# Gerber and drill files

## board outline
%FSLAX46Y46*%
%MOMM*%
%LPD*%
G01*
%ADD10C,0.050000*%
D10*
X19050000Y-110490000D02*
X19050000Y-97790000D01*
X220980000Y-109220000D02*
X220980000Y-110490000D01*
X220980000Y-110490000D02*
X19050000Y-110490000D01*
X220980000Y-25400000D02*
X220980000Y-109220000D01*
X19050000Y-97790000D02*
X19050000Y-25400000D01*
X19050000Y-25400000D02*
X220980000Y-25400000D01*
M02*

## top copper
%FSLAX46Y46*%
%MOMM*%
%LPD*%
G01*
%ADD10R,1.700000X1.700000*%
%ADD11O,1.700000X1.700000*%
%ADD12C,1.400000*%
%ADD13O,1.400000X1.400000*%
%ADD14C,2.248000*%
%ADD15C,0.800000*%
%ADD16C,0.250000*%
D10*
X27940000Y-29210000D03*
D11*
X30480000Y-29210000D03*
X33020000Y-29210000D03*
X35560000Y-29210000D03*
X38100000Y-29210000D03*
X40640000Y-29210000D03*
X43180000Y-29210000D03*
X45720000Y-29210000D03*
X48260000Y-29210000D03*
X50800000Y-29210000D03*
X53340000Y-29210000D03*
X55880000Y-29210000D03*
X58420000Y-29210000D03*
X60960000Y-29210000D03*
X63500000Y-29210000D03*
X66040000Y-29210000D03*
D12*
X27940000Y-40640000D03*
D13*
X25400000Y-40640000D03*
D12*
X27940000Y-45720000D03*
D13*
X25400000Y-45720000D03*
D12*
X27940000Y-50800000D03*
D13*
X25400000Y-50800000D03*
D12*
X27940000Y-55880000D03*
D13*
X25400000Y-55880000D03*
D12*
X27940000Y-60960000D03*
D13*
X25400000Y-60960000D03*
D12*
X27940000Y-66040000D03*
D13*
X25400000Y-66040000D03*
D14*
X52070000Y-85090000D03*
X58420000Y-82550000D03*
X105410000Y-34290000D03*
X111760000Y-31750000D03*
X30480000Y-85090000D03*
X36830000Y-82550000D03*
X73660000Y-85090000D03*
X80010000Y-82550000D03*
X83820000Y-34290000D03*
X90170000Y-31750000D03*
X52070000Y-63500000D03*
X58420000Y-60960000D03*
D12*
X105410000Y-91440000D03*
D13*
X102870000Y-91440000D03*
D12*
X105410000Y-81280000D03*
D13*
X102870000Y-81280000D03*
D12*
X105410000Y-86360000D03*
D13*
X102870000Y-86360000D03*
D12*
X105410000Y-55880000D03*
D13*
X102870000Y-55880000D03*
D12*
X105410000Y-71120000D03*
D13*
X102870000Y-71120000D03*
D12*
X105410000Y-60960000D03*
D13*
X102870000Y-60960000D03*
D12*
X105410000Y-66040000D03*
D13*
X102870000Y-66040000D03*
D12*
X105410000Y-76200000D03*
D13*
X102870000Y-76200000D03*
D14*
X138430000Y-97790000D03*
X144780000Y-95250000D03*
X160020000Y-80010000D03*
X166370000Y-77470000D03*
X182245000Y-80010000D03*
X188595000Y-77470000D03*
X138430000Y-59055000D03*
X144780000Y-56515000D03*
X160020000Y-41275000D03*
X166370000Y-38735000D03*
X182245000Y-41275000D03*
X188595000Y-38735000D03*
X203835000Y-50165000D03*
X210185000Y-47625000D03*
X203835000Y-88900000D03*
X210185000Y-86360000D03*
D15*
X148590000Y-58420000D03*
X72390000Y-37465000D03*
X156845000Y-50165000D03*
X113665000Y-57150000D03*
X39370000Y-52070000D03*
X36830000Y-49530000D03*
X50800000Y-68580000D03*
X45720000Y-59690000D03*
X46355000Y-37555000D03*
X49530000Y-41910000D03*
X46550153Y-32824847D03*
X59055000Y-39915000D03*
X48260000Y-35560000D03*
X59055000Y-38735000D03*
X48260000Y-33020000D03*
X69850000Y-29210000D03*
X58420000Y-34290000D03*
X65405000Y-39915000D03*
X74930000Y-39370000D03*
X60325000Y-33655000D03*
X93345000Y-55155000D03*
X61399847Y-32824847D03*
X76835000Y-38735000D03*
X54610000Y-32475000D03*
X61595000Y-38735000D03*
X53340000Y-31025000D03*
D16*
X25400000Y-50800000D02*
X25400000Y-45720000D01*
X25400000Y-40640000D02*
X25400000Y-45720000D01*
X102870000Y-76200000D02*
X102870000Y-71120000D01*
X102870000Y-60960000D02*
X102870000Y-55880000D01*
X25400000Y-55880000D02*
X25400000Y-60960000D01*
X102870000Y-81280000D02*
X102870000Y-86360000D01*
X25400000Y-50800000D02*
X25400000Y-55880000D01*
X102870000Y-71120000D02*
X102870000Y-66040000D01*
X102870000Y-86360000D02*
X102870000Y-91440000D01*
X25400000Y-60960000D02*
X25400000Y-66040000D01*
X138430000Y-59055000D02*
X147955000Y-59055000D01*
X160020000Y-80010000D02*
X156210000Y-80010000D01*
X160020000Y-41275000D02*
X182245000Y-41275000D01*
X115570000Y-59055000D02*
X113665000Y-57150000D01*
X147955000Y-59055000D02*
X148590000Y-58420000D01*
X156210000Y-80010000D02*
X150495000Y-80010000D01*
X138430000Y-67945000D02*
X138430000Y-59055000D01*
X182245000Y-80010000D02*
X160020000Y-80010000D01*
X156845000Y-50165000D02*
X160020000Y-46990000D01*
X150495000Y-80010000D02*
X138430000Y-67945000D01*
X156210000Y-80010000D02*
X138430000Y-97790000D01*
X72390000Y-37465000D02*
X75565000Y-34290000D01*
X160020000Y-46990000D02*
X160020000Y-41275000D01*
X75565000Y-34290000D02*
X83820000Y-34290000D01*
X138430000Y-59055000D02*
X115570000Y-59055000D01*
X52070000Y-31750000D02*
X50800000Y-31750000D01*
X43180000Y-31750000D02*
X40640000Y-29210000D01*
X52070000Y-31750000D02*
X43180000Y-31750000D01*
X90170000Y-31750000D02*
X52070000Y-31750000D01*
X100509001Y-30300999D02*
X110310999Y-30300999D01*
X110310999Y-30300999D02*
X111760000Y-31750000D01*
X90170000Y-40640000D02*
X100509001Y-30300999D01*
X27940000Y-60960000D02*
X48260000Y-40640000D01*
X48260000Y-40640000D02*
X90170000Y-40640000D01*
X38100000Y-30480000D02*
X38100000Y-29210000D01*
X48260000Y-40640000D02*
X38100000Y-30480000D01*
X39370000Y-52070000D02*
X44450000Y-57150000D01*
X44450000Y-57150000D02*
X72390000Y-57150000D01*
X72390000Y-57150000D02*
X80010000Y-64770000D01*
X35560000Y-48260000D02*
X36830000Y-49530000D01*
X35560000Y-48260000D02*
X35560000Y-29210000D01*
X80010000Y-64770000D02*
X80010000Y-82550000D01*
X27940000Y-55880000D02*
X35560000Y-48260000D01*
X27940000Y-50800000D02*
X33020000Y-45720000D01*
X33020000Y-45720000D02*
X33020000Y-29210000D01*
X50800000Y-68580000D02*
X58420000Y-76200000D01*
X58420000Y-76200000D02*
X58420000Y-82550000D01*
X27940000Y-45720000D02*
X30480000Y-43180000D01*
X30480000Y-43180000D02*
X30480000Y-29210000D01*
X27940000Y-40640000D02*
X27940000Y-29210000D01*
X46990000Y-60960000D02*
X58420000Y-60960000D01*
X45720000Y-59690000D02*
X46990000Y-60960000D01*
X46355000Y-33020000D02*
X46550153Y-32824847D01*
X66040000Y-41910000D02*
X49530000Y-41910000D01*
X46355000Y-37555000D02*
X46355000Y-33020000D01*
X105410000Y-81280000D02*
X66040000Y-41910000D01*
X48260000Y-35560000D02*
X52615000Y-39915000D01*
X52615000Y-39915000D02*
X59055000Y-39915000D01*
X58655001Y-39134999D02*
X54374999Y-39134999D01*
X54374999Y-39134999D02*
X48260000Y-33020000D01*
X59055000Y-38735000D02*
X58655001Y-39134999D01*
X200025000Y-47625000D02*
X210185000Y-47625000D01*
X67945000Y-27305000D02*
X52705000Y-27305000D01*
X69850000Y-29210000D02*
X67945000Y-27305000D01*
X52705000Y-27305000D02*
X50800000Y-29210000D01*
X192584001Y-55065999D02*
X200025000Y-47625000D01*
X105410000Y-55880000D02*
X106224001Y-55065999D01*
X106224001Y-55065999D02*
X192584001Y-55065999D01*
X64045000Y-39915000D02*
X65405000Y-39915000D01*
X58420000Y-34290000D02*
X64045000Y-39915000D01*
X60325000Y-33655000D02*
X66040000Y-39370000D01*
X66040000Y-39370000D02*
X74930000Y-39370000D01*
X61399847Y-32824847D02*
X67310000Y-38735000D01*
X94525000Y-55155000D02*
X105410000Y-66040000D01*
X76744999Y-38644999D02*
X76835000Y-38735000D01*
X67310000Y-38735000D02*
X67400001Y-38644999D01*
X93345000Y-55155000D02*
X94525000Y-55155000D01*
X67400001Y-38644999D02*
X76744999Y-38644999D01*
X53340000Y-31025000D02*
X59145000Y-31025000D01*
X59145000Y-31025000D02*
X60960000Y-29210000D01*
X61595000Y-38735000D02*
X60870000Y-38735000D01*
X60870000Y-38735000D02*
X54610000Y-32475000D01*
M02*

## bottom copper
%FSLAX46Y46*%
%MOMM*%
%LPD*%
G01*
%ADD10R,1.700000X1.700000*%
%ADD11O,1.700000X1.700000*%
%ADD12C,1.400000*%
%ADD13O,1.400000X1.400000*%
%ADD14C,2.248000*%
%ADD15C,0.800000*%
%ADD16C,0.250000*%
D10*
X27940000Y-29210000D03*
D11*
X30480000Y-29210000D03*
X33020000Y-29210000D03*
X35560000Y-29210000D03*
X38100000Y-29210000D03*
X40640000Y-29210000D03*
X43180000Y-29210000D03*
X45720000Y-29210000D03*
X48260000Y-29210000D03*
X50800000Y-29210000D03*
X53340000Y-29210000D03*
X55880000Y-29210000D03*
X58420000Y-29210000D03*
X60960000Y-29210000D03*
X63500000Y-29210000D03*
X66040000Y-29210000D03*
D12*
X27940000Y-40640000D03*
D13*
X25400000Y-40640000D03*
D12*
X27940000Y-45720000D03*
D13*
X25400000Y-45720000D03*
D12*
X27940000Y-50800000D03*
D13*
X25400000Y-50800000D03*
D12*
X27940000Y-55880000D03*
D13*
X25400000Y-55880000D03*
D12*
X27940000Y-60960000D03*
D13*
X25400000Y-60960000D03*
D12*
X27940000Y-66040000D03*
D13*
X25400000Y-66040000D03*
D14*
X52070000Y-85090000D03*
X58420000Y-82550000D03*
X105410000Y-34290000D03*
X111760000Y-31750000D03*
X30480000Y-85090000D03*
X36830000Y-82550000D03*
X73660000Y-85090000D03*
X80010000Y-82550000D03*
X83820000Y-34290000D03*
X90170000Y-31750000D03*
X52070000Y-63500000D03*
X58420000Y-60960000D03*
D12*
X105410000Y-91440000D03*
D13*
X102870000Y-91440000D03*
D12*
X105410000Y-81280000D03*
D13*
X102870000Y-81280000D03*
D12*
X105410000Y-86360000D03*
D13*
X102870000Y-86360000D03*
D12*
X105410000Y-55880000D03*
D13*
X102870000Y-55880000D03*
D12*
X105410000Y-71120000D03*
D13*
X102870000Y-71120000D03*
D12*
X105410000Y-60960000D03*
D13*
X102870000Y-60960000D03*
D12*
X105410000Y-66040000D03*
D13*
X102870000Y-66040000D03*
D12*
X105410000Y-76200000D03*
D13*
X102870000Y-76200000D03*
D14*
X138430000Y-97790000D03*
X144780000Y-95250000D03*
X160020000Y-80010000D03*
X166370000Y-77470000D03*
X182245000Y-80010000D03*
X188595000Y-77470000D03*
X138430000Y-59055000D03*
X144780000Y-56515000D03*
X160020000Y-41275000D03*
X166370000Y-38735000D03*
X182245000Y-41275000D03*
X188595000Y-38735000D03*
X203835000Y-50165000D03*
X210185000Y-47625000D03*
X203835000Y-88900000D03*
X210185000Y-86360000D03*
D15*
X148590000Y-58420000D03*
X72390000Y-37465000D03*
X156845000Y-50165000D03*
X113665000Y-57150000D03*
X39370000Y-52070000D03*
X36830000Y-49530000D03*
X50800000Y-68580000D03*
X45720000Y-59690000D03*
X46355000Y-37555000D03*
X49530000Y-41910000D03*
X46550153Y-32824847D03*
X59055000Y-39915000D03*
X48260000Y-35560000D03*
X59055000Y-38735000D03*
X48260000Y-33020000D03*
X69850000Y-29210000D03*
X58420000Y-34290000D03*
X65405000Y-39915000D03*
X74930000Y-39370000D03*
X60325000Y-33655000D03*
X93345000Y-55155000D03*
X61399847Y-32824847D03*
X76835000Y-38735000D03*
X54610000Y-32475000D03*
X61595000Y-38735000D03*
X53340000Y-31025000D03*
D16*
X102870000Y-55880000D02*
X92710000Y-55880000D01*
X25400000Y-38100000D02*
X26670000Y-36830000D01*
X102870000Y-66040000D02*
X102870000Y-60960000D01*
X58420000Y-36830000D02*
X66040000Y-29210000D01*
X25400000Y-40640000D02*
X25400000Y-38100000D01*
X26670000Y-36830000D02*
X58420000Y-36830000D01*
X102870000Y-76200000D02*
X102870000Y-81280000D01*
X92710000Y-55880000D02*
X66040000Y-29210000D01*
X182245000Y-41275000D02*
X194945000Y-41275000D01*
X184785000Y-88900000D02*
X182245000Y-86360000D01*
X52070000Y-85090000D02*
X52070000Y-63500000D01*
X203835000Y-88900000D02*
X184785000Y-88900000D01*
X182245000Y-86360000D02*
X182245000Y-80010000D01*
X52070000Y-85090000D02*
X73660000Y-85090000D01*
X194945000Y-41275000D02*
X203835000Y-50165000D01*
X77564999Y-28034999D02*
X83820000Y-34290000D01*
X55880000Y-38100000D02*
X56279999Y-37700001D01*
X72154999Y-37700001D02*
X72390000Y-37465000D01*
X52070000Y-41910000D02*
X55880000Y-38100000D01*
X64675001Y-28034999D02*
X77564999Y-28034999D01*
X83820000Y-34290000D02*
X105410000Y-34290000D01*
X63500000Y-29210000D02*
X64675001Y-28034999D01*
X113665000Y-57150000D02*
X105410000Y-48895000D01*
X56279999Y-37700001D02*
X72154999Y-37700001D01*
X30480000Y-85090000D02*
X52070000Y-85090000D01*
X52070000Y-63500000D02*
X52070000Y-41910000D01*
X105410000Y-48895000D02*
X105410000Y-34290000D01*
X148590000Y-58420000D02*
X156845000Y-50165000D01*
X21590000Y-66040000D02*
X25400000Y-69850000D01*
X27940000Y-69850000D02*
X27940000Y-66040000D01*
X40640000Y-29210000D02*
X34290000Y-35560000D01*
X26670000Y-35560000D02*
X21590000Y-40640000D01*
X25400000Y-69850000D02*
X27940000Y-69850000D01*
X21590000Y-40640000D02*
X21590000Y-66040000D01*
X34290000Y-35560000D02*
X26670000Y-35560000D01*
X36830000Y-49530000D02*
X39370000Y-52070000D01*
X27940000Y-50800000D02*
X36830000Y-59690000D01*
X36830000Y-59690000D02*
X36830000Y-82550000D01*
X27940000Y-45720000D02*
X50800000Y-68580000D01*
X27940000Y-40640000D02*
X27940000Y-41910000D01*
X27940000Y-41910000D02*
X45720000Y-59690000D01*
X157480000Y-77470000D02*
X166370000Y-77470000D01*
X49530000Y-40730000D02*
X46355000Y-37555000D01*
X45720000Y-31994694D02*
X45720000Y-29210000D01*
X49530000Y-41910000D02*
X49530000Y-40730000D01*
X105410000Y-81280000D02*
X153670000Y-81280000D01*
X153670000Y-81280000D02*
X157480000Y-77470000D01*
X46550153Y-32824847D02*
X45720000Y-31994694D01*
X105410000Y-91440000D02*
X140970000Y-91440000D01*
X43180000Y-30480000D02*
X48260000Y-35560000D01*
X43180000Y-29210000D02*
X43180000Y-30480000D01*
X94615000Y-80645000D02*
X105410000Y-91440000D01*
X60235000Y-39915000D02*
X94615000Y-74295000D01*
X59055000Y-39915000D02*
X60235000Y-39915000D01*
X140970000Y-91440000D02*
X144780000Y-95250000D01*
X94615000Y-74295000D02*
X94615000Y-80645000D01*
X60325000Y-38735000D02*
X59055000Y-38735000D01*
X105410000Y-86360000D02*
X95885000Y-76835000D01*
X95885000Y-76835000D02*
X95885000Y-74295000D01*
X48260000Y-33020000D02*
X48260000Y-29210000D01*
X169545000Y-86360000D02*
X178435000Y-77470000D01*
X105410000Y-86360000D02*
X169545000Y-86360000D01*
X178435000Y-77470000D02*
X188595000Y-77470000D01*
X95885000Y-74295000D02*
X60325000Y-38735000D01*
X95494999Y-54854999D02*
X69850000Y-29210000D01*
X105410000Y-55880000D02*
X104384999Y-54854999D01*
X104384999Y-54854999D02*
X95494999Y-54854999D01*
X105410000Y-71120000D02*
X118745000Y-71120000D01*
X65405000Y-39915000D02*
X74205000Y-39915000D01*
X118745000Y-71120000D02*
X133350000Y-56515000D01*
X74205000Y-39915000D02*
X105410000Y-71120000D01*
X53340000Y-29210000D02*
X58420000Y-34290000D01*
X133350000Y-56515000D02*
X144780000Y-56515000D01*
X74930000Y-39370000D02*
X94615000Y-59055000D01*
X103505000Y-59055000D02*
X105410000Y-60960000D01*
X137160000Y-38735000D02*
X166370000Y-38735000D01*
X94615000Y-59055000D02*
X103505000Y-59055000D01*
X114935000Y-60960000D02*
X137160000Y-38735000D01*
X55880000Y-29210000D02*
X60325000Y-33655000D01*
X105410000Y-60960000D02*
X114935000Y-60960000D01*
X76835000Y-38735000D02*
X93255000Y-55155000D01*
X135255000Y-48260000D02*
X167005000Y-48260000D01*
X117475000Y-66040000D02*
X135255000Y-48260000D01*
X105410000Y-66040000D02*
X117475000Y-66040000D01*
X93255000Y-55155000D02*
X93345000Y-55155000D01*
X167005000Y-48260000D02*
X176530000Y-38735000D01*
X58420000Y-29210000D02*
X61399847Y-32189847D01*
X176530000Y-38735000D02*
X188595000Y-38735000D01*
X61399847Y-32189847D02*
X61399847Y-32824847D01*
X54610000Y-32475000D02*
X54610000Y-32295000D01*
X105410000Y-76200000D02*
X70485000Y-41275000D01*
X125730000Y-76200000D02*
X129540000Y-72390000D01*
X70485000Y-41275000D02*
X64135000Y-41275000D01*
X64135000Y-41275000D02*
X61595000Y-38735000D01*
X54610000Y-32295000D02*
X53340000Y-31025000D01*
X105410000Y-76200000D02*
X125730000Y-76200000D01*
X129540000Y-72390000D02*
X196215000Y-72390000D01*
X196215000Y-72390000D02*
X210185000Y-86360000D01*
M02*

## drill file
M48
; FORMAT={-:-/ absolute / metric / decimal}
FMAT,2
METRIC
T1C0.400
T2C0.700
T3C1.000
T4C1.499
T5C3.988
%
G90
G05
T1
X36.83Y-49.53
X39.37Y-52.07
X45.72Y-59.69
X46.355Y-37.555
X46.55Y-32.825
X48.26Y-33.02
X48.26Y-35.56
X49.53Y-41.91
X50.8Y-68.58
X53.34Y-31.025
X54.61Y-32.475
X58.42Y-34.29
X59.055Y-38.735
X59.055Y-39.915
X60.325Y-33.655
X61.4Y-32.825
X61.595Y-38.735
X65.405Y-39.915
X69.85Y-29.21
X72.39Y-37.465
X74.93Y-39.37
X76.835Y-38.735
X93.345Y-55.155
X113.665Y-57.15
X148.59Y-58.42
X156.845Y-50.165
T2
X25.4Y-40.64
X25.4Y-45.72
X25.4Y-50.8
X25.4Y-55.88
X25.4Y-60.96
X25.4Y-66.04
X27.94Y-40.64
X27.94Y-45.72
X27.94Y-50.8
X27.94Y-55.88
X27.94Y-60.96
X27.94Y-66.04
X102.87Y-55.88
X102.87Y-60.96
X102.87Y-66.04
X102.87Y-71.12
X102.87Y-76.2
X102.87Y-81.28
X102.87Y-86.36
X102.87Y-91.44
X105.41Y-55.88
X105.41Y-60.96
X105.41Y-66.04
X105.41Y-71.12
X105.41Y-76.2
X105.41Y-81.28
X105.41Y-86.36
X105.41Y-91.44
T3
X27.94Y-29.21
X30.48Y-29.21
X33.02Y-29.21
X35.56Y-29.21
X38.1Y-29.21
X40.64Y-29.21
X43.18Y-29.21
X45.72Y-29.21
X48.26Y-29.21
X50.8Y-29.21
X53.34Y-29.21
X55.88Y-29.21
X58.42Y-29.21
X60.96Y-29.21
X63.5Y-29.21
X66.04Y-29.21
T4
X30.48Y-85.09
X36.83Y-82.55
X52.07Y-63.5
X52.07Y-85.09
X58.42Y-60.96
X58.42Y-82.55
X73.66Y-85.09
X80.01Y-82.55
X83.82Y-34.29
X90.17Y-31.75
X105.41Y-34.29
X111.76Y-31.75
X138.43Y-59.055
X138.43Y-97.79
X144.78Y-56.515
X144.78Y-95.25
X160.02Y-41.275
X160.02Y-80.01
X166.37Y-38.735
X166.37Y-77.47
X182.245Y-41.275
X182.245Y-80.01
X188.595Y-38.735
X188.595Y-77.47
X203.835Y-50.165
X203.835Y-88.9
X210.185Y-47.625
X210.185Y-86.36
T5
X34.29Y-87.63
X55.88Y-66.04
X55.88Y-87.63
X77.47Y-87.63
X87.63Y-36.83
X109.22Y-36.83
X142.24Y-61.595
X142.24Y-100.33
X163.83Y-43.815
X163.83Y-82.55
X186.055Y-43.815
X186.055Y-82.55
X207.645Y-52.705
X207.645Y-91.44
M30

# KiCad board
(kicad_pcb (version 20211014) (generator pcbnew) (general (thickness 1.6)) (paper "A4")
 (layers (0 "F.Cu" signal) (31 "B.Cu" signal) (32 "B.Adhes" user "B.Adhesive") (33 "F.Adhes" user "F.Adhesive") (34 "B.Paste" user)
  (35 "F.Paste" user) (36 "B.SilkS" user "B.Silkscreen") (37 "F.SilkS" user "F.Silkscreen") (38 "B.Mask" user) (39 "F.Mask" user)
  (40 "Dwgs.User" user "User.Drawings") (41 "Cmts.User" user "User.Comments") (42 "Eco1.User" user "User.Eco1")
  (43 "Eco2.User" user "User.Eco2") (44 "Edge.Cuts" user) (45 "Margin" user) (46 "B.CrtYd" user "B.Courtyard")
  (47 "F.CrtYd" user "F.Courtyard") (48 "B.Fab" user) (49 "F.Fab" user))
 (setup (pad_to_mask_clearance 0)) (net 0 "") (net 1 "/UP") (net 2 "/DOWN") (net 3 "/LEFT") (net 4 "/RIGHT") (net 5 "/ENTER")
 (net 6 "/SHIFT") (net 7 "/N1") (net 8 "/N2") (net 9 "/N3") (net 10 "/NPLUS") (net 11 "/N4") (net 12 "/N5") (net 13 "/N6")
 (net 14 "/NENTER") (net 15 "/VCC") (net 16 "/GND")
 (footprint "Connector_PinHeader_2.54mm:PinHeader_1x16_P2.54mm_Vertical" (layer "F.Cu") (at 27.94 29.21 90)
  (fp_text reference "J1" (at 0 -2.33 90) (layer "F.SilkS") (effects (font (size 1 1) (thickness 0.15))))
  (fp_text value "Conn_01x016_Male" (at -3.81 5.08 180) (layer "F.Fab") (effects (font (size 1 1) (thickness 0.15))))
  (pad "1" thru_hole rect locked (at 0 0 90) (size 1.7 1.7) (drill 1) (layers *.Cu *.Mask) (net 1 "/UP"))
  (pad "2" thru_hole oval locked (at 0 2.54 90) (size 1.7 1.7) (drill 1) (layers *.Cu *.Mask) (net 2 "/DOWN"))
  (pad "3" thru_hole oval locked (at 0 5.08 90) (size 1.7 1.7) (drill 1) (layers *.Cu *.Mask) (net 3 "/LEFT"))
  (pad "4" thru_hole oval locked (at 0 7.62 90) (size 1.7 1.7) (drill 1) (layers *.Cu *.Mask) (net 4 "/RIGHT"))
  (pad "5" thru_hole oval locked (at 0 10.16 90) (size 1.7 1.7) (drill 1) (layers *.Cu *.Mask) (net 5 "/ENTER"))
  (pad "6" thru_hole oval locked (at 0 12.7 90) (size 1.7 1.7) (drill 1) (layers *.Cu *.Mask) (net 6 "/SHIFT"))
  (pad "7" thru_hole oval locked (at 0 15.24 90) (size 1.7 1.7) (drill 1) (layers *.Cu *.Mask) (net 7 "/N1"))
  (pad "8" thru_hole oval locked (at 0 17.78 90) (size 1.7 1.7) (drill 1) (layers *.Cu *.Mask) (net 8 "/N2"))
  (pad "9" thru_hole oval locked (at 0 20.32 90) (size 1.7 1.7) (drill 1) (layers *.Cu *.Mask) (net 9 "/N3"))
  (pad "10" thru_hole oval locked (at 0 22.86 90) (size 1.7 1.7) (drill 1) (layers *.Cu *.Mask) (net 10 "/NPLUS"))
  (pad "11" thru_hole oval locked (at 0 25.4 90) (size 1.7 1.7) (drill 1) (layers *.Cu *.Mask) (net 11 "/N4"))
  (pad "12" thru_hole oval locked (at 0 27.94 90) (size 1.7 1.7) (drill 1) (layers *.Cu *.Mask) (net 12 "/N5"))
  (pad "13" thru_hole oval locked (at 0 30.48 90) (size 1.7 1.7) (drill 1) (layers *.Cu *.Mask) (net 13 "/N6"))
  (pad "14" thru_hole oval locked (at 0 33.02 90) (size 1.7 1.7) (drill 1) (layers *.Cu *.Mask) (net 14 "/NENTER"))
  (pad "15" thru_hole oval locked (at 0 35.56 90) (size 1.7 1.7) (drill 1) (layers *.Cu *.Mask) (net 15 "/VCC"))
  (pad "16" thru_hole oval locked (at 0 38.1 90) (size 1.7 1.7) (drill 1) (layers *.Cu *.Mask) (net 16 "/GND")))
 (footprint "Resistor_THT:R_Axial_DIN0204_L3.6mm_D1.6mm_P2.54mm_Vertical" (layer "F.Cu") (at 27.94 40.64 180)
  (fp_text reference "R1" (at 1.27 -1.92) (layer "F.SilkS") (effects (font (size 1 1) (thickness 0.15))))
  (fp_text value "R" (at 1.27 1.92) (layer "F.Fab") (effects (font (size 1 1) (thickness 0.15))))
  (pad "1" thru_hole circle locked (at 0 0 180) (size 1.4 1.4) (drill 0.7) (layers *.Cu *.Mask) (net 1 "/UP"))
  (pad "2" thru_hole oval locked (at 2.54 0 180) (size 1.4 1.4) (drill 0.7) (layers *.Cu *.Mask) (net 16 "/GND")))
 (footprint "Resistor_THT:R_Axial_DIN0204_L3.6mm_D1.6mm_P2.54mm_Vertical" (layer "F.Cu") (at 27.94 45.72 180)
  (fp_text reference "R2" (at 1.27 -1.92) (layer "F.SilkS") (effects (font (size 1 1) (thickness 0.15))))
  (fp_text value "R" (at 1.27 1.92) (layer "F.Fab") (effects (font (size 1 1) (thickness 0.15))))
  (pad "1" thru_hole circle locked (at 0 0 180) (size 1.4 1.4) (drill 0.7) (layers *.Cu *.Mask) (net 2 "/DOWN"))
  (pad "2" thru_hole oval locked (at 2.54 0 180) (size 1.4 1.4) (drill 0.7) (layers *.Cu *.Mask) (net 16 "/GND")))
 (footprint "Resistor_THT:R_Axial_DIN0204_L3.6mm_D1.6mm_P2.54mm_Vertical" (layer "F.Cu") (at 27.94 50.8 180)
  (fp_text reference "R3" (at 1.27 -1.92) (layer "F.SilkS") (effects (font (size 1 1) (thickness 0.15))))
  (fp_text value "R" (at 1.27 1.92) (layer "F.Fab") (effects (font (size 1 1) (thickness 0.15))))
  (pad "1" thru_hole circle locked (at 0 0 180) (size 1.4 1.4) (drill 0.7) (layers *.Cu *.Mask) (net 3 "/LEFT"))
  (pad "2" thru_hole oval locked (at 2.54 0 180) (size 1.4 1.4) (drill 0.7) (layers *.Cu *.Mask) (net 16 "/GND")))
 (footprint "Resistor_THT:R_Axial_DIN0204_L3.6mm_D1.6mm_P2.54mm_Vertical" (layer "F.Cu") (at 27.94 55.88 180)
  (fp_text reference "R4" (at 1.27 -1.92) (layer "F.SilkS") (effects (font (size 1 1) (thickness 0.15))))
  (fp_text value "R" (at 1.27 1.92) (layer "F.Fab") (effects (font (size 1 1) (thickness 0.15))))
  (pad "1" thru_hole circle locked (at 0 0 180) (size 1.4 1.4) (drill 0.7) (layers *.Cu *.Mask) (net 4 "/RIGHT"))
  (pad "2" thru_hole oval locked (at 2.54 0 180) (size 1.4 1.4) (drill 0.7) (layers *.Cu *.Mask) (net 16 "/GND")))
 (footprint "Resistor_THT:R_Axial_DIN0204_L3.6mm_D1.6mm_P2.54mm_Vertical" (layer "F.Cu") (at 27.94 60.96 180)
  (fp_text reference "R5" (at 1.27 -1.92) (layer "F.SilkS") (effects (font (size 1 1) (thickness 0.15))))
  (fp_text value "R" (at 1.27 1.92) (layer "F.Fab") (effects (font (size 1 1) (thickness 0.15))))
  (pad "1" thru_hole circle locked (at 0 0 180) (size 1.4 1.4) (drill 0.7) (layers *.Cu *.Mask) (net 5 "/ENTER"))
  (pad "2" thru_hole oval locked (at 2.54 0 180) (size 1.4 1.4) (drill 0.7) (layers *.Cu *.Mask) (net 16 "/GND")))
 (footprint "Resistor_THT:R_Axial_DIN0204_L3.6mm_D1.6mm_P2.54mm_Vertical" (layer "F.Cu") (at 27.94 66.04 180)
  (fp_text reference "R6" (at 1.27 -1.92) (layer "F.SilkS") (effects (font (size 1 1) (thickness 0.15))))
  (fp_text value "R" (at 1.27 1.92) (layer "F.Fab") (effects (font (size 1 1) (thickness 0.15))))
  (pad "1" thru_hole circle locked (at 0 0 180) (size 1.4 1.4) (drill 0.7) (layers *.Cu *.Mask) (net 6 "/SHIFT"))
  (pad "2" thru_hole oval locked (at 2.54 0 180) (size 1.4 1.4) (drill 0.7) (layers *.Cu *.Mask) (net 16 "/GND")))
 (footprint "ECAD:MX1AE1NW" (layer "F.Cu") (at 52.07 85.09)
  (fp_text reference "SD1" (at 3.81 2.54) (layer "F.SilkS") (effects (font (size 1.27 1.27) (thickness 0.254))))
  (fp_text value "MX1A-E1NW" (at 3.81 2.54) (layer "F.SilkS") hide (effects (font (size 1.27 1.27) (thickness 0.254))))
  (pad "" np_thru_hole circle locked (at 3.81 2.54) (size 3.9878 0) (drill 3.9878) (layers *.Cu *.Mask))
  (pad "1" thru_hole circle locked (at 0 0) (size 2.248 2.248) (drill 1.4986) (layers *.Cu *.Mask) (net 15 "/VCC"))
  (pad "2" thru_hole circle locked (at 6.35 -2.54) (size 2.248 2.248) (drill 1.4986) (layers *.Cu *.Mask) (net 2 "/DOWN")))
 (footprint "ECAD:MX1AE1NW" (layer "F.Cu") (at 105.41 34.29)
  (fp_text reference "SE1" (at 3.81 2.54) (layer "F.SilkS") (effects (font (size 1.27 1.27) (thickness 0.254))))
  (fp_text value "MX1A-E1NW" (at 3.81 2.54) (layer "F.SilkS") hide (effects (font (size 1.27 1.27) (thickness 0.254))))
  (pad "" np_thru_hole circle locked (at 3.81 2.54) (size 3.9878 0) (drill 3.9878) (layers *.Cu *.Mask))
  (pad "1" thru_hole circle locked (at 0 0) (size 2.248 2.248) (drill 1.4986) (layers *.Cu *.Mask) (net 15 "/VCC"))
  (pad "2" thru_hole circle locked (at 6.35 -2.54) (size 2.248 2.248) (drill 1.4986) (layers *.Cu *.Mask) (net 5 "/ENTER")))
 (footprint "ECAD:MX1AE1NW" (layer "F.Cu") (at 30.48 85.09)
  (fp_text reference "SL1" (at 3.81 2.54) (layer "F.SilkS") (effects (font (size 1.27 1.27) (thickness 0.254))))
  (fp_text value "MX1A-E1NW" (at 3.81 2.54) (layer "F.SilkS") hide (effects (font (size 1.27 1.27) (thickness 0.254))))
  (pad "" np_thru_hole circle locked (at 3.81 2.54) (size 3.9878 0) (drill 3.9878) (layers *.Cu *.Mask))
  (pad "1" thru_hole circle locked (at 0 0) (size 2.248 2.248) (drill 1.4986) (layers *.Cu *.Mask) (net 15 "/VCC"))
  (pad "2" thru_hole circle locked (at 6.35 -2.54) (size 2.248 2.248) (drill 1.4986) (layers *.Cu *.Mask) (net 3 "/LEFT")))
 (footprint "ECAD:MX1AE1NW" (layer "F.Cu") (at 73.66 85.09)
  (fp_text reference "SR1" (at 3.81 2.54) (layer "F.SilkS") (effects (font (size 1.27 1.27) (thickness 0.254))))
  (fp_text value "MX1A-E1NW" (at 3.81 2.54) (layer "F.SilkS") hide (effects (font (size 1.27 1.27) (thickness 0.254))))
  (pad "" np_thru_hole circle locked (at 3.81 2.54) (size 3.9878 0) (drill 3.9878) (layers *.Cu *.Mask))
  (pad "1" thru_hole circle locked (at 0 0) (size 2.248 2.248) (drill 1.4986) (layers *.Cu *.Mask) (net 15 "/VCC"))
  (pad "2" thru_hole circle locked (at 6.35 -2.54) (size 2.248 2.248) (drill 1.4986) (layers *.Cu *.Mask) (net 4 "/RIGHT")))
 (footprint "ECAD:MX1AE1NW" (layer "F.Cu") (at 83.82 34.29)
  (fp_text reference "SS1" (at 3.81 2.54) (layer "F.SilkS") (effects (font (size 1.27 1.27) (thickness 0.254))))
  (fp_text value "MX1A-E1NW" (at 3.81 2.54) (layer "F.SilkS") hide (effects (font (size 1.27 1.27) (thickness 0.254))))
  (pad "" np_thru_hole circle locked (at 3.81 2.54) (size 3.9878 0) (drill 3.9878) (layers *.Cu *.Mask))
  (pad "1" thru_hole circle locked (at 0 0) (size 2.248 2.248) (drill 1.4986) (layers *.Cu *.Mask) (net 15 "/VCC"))
  (pad "2" thru_hole circle locked (at 6.35 -2.54) (size 2.248 2.248) (drill 1.4986) (layers *.Cu *.Mask) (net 6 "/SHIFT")))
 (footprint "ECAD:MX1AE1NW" (layer "F.Cu") (at 52.07 63.5)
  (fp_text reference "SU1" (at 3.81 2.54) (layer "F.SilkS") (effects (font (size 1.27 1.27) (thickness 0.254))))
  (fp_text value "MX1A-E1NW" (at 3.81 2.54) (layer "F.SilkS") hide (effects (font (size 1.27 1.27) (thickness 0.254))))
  (pad "" np_thru_hole circle locked (at 3.81 2.54) (size 3.9878 0) (drill 3.9878) (layers *.Cu *.Mask))
  (pad "1" thru_hole circle locked (at 0 0) (size 2.248 2.248) (drill 1.4986) (layers *.Cu *.Mask) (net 15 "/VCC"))
  (pad "2" thru_hole circle locked (at 6.35 -2.54) (size 2.248 2.248) (drill 1.4986) (layers *.Cu *.Mask) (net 1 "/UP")))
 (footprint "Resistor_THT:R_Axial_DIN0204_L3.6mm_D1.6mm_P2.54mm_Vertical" (layer "F.Cu") (at 105.41 91.44 180)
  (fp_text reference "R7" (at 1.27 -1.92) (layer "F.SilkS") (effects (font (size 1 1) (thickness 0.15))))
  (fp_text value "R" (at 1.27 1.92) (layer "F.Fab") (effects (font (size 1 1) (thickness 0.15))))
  (pad "1" thru_hole circle locked (at 0 0 180) (size 1.4 1.4) (drill 0.7) (layers *.Cu *.Mask) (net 7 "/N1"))
  (pad "2" thru_hole oval locked (at 2.54 0 180) (size 1.4 1.4) (drill 0.7) (layers *.Cu *.Mask) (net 16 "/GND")))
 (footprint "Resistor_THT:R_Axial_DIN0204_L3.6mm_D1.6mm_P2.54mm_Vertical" (layer "F.Cu") (at 105.41 81.28 180)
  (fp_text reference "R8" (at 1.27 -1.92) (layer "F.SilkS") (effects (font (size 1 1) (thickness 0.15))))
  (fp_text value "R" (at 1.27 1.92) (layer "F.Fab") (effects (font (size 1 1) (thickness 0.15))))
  (pad "1" thru_hole circle locked (at 0 0 180) (size 1.4 1.4) (drill 0.7) (layers *.Cu *.Mask) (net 8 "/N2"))
  (pad "2" thru_hole oval locked (at 2.54 0 180) (size 1.4 1.4) (drill 0.7) (layers *.Cu *.Mask) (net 16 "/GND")))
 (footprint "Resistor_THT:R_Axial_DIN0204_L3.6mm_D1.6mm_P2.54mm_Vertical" (layer "F.Cu") (at 105.41 86.36 180)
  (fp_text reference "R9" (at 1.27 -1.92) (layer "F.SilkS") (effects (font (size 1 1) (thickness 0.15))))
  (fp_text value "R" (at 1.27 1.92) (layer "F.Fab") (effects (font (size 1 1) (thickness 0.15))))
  (pad "1" thru_hole circle locked (at 0 0 180) (size 1.4 1.4) (drill 0.7) (layers *.Cu *.Mask) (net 9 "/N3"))
  (pad "2" thru_hole oval locked (at 2.54 0 180) (size 1.4 1.4) (drill 0.7) (layers *.Cu *.Mask) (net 16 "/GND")))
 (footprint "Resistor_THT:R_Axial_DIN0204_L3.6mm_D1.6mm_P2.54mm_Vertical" (layer "F.Cu") (at 105.41 55.88 180)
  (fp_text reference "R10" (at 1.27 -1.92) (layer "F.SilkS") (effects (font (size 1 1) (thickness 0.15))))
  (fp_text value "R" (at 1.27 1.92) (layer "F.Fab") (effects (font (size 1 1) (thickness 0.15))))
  (pad "1" thru_hole circle locked (at 0 0 180) (size 1.4 1.4) (drill 0.7) (layers *.Cu *.Mask) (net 10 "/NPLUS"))
  (pad "2" thru_hole oval locked (at 2.54 0 180) (size 1.4 1.4) (drill 0.7) (layers *.Cu *.Mask) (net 16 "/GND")))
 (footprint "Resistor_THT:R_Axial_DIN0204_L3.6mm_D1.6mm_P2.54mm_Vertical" (layer "F.Cu") (at 105.41 71.12 180)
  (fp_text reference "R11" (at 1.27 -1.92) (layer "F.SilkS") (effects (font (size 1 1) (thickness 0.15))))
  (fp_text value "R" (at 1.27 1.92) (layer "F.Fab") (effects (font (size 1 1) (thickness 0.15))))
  (pad "1" thru_hole circle locked (at 0 0 180) (size 1.4 1.4) (drill 0.7) (layers *.Cu *.Mask) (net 11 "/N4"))
  (pad "2" thru_hole oval locked (at 2.54 0 180) (size 1.4 1.4) (drill 0.7) (layers *.Cu *.Mask) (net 16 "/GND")))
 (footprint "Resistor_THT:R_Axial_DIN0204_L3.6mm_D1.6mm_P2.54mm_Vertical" (layer "F.Cu") (at 105.41 60.96 180)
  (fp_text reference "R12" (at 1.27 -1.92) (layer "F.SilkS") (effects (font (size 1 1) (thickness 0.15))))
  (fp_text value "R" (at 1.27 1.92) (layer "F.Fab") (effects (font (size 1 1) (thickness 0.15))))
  (pad "1" thru_hole circle locked (at 0 0 180) (size 1.4 1.4) (drill 0.7) (layers *.Cu *.Mask) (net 12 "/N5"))
  (pad "2" thru_hole oval locked (at 2.54 0 180) (size 1.4 1.4) (drill 0.7) (layers *.Cu *.Mask) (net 16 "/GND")))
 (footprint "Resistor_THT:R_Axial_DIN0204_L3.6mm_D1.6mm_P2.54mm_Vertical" (layer "F.Cu") (at 105.41 66.04 180)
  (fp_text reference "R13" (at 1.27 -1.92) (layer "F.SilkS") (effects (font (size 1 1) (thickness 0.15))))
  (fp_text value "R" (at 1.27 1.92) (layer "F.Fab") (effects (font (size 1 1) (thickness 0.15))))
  (pad "1" thru_hole circle locked (at 0 0 180) (size 1.4 1.4) (drill 0.7) (layers *.Cu *.Mask) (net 13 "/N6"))
  (pad "2" thru_hole oval locked (at 2.54 0 180) (size 1.4 1.4) (drill 0.7) (layers *.Cu *.Mask) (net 16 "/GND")))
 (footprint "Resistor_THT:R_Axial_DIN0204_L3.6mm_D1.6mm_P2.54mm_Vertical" (layer "F.Cu") (at 105.41 76.2 180)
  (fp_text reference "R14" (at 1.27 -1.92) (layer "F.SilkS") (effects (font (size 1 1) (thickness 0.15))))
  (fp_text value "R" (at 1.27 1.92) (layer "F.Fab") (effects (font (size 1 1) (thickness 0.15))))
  (pad "1" thru_hole circle locked (at 0 0 180) (size 1.4 1.4) (drill 0.7) (layers *.Cu *.Mask) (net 14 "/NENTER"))
  (pad "2" thru_hole oval locked (at 2.54 0 180) (size 1.4 1.4) (drill 0.7) (layers *.Cu *.Mask) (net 16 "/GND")))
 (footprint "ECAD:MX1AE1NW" (layer "F.Cu") (at 138.43 97.79)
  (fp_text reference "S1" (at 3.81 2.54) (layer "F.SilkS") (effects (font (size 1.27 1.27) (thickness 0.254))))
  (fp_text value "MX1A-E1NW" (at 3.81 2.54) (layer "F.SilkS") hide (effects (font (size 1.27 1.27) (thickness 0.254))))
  (pad "" np_thru_hole circle locked (at 3.81 2.54) (size 3.9878 0) (drill 3.9878) (layers *.Cu *.Mask))
  (pad "1" thru_hole circle locked (at 0 0) (size 2.248 2.248) (drill 1.4986) (layers *.Cu *.Mask) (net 15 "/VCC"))
  (pad "2" thru_hole circle locked (at 6.35 -2.54) (size 2.248 2.248) (drill 1.4986) (layers *.Cu *.Mask) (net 7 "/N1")))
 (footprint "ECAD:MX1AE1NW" (layer "F.Cu") (at 160.02 80.01)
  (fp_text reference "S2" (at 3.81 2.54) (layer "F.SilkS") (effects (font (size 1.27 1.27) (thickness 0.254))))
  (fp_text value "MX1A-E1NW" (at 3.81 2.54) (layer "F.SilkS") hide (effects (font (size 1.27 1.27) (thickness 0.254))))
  (pad "" np_thru_hole circle locked (at 3.81 2.54) (size 3.9878 0) (drill 3.9878) (layers *.Cu *.Mask))
  (pad "1" thru_hole circle locked (at 0 0) (size 2.248 2.248) (drill 1.4986) (layers *.Cu *.Mask) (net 15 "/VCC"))
  (pad "2" thru_hole circle locked (at 6.35 -2.54) (size 2.248 2.248) (drill 1.4986) (layers *.Cu *.Mask) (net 8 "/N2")))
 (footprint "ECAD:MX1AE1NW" (layer "F.Cu") (at 182.245 80.01)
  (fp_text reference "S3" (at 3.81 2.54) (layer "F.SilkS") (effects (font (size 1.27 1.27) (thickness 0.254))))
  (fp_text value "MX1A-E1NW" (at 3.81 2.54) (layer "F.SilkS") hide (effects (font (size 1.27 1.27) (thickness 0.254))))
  (pad "" np_thru_hole circle locked (at 3.81 2.54) (size 3.9878 0) (drill 3.9878) (layers *.Cu *.Mask))
  (pad "1" thru_hole circle locked (at 0 0) (size 2.248 2.248) (drill 1.4986) (layers *.Cu *.Mask) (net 15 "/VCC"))
  (pad "2" thru_hole circle locked (at 6.35 -2.54) (size 2.248 2.248) (drill 1.4986) (layers *.Cu *.Mask) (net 9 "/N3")))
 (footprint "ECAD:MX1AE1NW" (layer "F.Cu") (at 138.43 59.055)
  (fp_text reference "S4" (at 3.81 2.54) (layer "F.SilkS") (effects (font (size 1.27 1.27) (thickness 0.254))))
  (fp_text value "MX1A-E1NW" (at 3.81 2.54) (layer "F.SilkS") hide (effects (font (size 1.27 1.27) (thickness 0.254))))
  (pad "" np_thru_hole circle locked (at 3.81 2.54) (size 3.9878 0) (drill 3.9878) (layers *.Cu *.Mask))
  (pad "1" thru_hole circle locked (at 0 0) (size 2.248 2.248) (drill 1.4986) (layers *.Cu *.Mask) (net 15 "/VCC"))
  (pad "2" thru_hole circle locked (at 6.35 -2.54) (size 2.248 2.248) (drill 1.4986) (layers *.Cu *.Mask) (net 11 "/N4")))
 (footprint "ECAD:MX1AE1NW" (layer "F.Cu") (at 160.02 41.275)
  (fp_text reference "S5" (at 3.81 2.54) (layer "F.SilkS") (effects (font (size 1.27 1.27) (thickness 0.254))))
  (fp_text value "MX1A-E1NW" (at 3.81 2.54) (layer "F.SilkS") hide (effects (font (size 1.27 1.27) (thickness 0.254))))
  (pad "" np_thru_hole circle locked (at 3.81 2.54) (size 3.9878 0) (drill 3.9878) (layers *.Cu *.Mask))
  (pad "1" thru_hole circle locked (at 0 0) (size 2.248 2.248) (drill 1.4986) (layers *.Cu *.Mask) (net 15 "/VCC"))
  (pad "2" thru_hole circle locked (at 6.35 -2.54) (size 2.248 2.248) (drill 1.4986) (layers *.Cu *.Mask) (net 12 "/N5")))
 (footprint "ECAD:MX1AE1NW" (layer "F.Cu") (at 182.245 41.275)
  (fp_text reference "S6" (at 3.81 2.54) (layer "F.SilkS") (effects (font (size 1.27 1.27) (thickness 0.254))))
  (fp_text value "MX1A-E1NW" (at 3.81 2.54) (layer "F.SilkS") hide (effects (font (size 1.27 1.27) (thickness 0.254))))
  (pad "" np_thru_hole circle locked (at 3.81 2.54) (size 3.9878 0) (drill 3.9878) (layers *.Cu *.Mask))
  (pad "1" thru_hole circle locked (at 0 0) (size 2.248 2.248) (drill 1.4986) (layers *.Cu *.Mask) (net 15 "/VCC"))
  (pad "2" thru_hole circle locked (at 6.35 -2.54) (size 2.248 2.248) (drill 1.4986) (layers *.Cu *.Mask) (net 13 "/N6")))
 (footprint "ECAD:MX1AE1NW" (layer "F.Cu") (at 203.835 50.165)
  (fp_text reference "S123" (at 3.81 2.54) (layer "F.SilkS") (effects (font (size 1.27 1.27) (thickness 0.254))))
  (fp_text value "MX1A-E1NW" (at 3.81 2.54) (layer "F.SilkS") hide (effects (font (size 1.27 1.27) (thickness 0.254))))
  (pad "" np_thru_hole circle locked (at 3.81 2.54) (size 3.9878 0) (drill 3.9878) (layers *.Cu *.Mask))
  (pad "1" thru_hole circle locked (at 0 0) (size 2.248 2.248) (drill 1.4986) (layers *.Cu *.Mask) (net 15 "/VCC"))
  (pad "2" thru_hole circle locked (at 6.35 -2.54) (size 2.248 2.248) (drill 1.4986) (layers *.Cu *.Mask) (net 10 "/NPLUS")))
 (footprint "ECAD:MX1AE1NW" (layer "F.Cu") (at 203.835 88.9)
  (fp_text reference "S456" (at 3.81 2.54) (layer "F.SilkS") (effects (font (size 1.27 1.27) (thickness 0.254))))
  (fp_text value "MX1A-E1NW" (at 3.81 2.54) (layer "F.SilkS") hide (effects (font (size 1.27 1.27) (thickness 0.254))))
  (pad "" np_thru_hole circle locked (at 3.81 2.54) (size 3.9878 0) (drill 3.9878) (layers *.Cu *.Mask))
  (pad "1" thru_hole circle locked (at 0 0) (size 2.248 2.248) (drill 1.4986) (layers *.Cu *.Mask) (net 15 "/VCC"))
  (pad "2" thru_hole circle locked (at 6.35 -2.54) (size 2.248 2.248) (drill 1.4986) (layers *.Cu *.Mask) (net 14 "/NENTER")))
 (gr_line (start 19.05 110.49) (end 19.05 97.79) (layer "Edge.Cuts") (width 0.05))
 (gr_line (start 220.98 109.22) (end 220.98 110.49) (layer "Edge.Cuts") (width 0.05))
 (gr_line (start 220.98 110.49) (end 19.05 110.49) (layer "Edge.Cuts") (width 0.05))
 (gr_line (start 220.98 25.4) (end 220.98 109.22) (layer "Edge.Cuts") (width 0.05))
 (gr_line (start 19.05 97.79) (end 19.05 25.4) (layer "Edge.Cuts") (width 0.05))
 (gr_line (start 19.05 25.4) (end 220.98 25.4) (layer "Edge.Cuts") (width 0.05))
 (segment (start 25.4 50.8) (end 25.4 45.72) (width 0.25) (layer "F.Cu") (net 16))
 (segment (start 25.4 40.64) (end 25.4 45.72) (width 0.25) (layer "F.Cu") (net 16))
 (segment (start 102.87 76.2) (end 102.87 71.12) (width 0.25) (layer "F.Cu") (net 16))
 (segment (start 102.87 60.96) (end 102.87 55.88) (width 0.25) (layer "F.Cu") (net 16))
 (segment (start 25.4 55.88) (end 25.4 60.96) (width 0.25) (layer "F.Cu") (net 16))
 (segment (start 102.87 81.28) (end 102.87 86.36) (width 0.25) (layer "F.Cu") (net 16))
 (segment (start 25.4 50.8) (end 25.4 55.88) (width 0.25) (layer "F.Cu") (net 16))
 (segment (start 102.87 71.12) (end 102.87 66.04) (width 0.25) (layer "F.Cu") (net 16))
 (segment (start 102.87 86.36) (end 102.87 91.44) (width 0.25) (layer "F.Cu") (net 16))
 (segment (start 25.4 60.96) (end 25.4 66.04) (width 0.25) (layer "F.Cu") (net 16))
 (segment (start 102.87 55.88) (end 92.71 55.88) (width 0.25) (layer "B.Cu") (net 16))
 (segment (start 25.4 38.1) (end 26.67 36.83) (width 0.25) (layer "B.Cu") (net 16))
 (segment (start 102.87 66.04) (end 102.87 60.96) (width 0.25) (layer "B.Cu") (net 16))
 (segment (start 58.42 36.83) (end 66.04 29.21) (width 0.25) (layer "B.Cu") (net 16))
 (segment (start 25.4 40.64) (end 25.4 38.1) (width 0.25) (layer "B.Cu") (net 16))
 (segment (start 26.67 36.83) (end 58.42 36.83) (width 0.25) (layer "B.Cu") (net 16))
 (segment (start 102.87 76.2) (end 102.87 81.28) (width 0.25) (layer "B.Cu") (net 16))
 (segment (start 92.71 55.88) (end 66.04 29.21) (width 0.25) (layer "B.Cu") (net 16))
 (segment (start 138.43 59.055) (end 147.955 59.055) (width 0.25) (layer "F.Cu") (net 15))
 (segment (start 160.02 80.01) (end 156.21 80.01) (width 0.25) (layer "F.Cu") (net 15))
 (segment (start 160.02 41.275) (end 182.245 41.275) (width 0.25) (layer "F.Cu") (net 15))
 (segment (start 115.57 59.055) (end 113.665 57.15) (width 0.25) (layer "F.Cu") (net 15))
 (segment (start 147.955 59.055) (end 148.59 58.42) (width 0.25) (layer "F.Cu") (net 15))
 (segment (start 156.21 80.01) (end 150.495 80.01) (width 0.25) (layer "F.Cu") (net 15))
 (segment (start 138.43 67.945) (end 138.43 59.055) (width 0.25) (layer "F.Cu") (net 15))
 (segment (start 182.245 80.01) (end 160.02 80.01) (width 0.25) (layer "F.Cu") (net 15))
 (segment (start 156.845 50.165) (end 160.02 46.99) (width 0.25) (layer "F.Cu") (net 15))
 (segment (start 150.495 80.01) (end 138.43 67.945) (width 0.25) (layer "F.Cu") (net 15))
 (segment (start 156.21 80.01) (end 138.43 97.79) (width 0.25) (layer "F.Cu") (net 15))
 (segment (start 72.39 37.465) (end 75.565 34.29) (width 0.25) (layer "F.Cu") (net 15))
 (segment (start 160.02 46.99) (end 160.02 41.275) (width 0.25) (layer "F.Cu") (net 15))
 (segment (start 75.565 34.29) (end 83.82 34.29) (width 0.25) (layer "F.Cu") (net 15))
 (segment (start 138.43 59.055) (end 115.57 59.055) (width 0.25) (layer "F.Cu") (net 15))
 (via (at 148.59 58.42) (size 0.8) (drill 0.4) (layers "F.Cu" "B.Cu") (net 15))
 (via (at 72.39 37.465) (size 0.8) (drill 0.4) (layers "F.Cu" "B.Cu") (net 15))
 (via (at 156.845 50.165) (size 0.8) (drill 0.4) (layers "F.Cu" "B.Cu") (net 15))
 (via (at 113.665 57.15) (size 0.8) (drill 0.4) (layers "F.Cu" "B.Cu") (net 15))
 (segment (start 182.245 41.275) (end 194.945 41.275) (width 0.25) (layer "B.Cu") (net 15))
 (segment (start 184.785 88.9) (end 182.245 86.36) (width 0.25) (layer "B.Cu") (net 15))
 (segment (start 52.07 85.09) (end 52.07 63.5) (width 0.25) (layer "B.Cu") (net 15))
 (segment (start 203.835 88.9) (end 184.785 88.9) (width 0.25) (layer "B.Cu") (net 15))
 (segment (start 182.245 86.36) (end 182.245 80.01) (width 0.25) (layer "B.Cu") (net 15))
 (segment (start 52.07 85.09) (end 73.66 85.09) (width 0.25) (layer "B.Cu") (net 15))
 (segment (start 194.945 41.275) (end 203.835 50.165) (width 0.25) (layer "B.Cu") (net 15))
 (segment (start 77.564999 28.034999) (end 83.82 34.29) (width 0.25) (layer "B.Cu") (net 15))
 (segment (start 55.88 38.1) (end 56.279999 37.700001) (width 0.25) (layer "B.Cu") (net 15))
 (segment (start 72.154999 37.700001) (end 72.39 37.465) (width 0.25) (layer "B.Cu") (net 15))
 (segment (start 52.07 41.91) (end 55.88 38.1) (width 0.25) (layer "B.Cu") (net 15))
 (segment (start 64.675001 28.034999) (end 77.564999 28.034999) (width 0.25) (layer "B.Cu") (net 15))
 (segment (start 83.82 34.29) (end 105.41 34.29) (width 0.25) (layer "B.Cu") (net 15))
 (segment (start 63.5 29.21) (end 64.675001 28.034999) (width 0.25) (layer "B.Cu") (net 15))
 (segment (start 113.665 57.15) (end 105.41 48.895) (width 0.25) (layer "B.Cu") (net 15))
 (segment (start 56.279999 37.700001) (end 72.154999 37.700001) (width 0.25) (layer "B.Cu") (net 15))
 (segment (start 30.48 85.09) (end 52.07 85.09) (width 0.25) (layer "B.Cu") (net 15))
 (segment (start 52.07 63.5) (end 52.07 41.91) (width 0.25) (layer "B.Cu") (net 15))
 (segment (start 105.41 48.895) (end 105.41 34.29) (width 0.25) (layer "B.Cu") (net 15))
 (segment (start 148.59 58.42) (end 156.845 50.165) (width 0.25) (layer "B.Cu") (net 15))
 (segment (start 52.07 31.75) (end 50.8 31.75) (width 0.25) (layer "F.Cu") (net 6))
 (segment (start 43.18 31.75) (end 40.64 29.21) (width 0.25) (layer "F.Cu") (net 6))
 (segment (start 52.07 31.75) (end 43.18 31.75) (width 0.25) (layer "F.Cu") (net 6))
 (segment (start 90.17 31.75) (end 52.07 31.75) (width 0.25) (layer "F.Cu") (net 6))
 (segment (start 21.59 66.04) (end 25.4 69.85) (width 0.25) (layer "B.Cu") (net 6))
 (segment (start 27.94 69.85) (end 27.94 66.04) (width 0.25) (layer "B.Cu") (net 6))
 (segment (start 40.64 29.21) (end 34.29 35.56) (width 0.25) (layer "B.Cu") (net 6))
 (segment (start 26.67 35.56) (end 21.59 40.64) (width 0.25) (layer "B.Cu") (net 6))
 (segment (start 25.4 69.85) (end 27.94 69.85) (width 0.25) (layer "B.Cu") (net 6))
 (segment (start 21.59 40.64) (end 21.59 66.04) (width 0.25) (layer "B.Cu") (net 6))
 (segment (start 34.29 35.56) (end 26.67 35.56) (width 0.25) (layer "B.Cu") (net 6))
 (segment (start 100.509001 30.300999) (end 110.310999 30.300999) (width 0.25) (layer "F.Cu") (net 5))
 (segment (start 110.310999 30.300999) (end 111.76 31.75) (width 0.25) (layer "F.Cu") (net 5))
 (segment (start 90.17 40.64) (end 100.509001 30.300999) (width 0.25) (layer "F.Cu") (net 5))
 (segment (start 27.94 60.96) (end 48.26 40.64) (width 0.25) (layer "F.Cu") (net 5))
 (segment (start 48.26 40.64) (end 90.17 40.64) (width 0.25) (layer "F.Cu") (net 5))
 (segment (start 38.1 30.48) (end 38.1 29.21) (width 0.25) (layer "F.Cu") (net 5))
 (segment (start 48.26 40.64) (end 38.1 30.48) (width 0.25) (layer "F.Cu") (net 5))
 (segment (start 39.37 52.07) (end 44.45 57.15) (width 0.25) (layer "F.Cu") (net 4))
 (segment (start 44.45 57.15) (end 72.39 57.15) (width 0.25) (layer "F.Cu") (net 4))
 (segment (start 72.39 57.15) (end 80.01 64.77) (width 0.25) (layer "F.Cu") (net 4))
 (segment (start 35.56 48.26) (end 36.83 49.53) (width 0.25) (layer "F.Cu") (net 4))
 (segment (start 35.56 48.26) (end 35.56 29.21) (width 0.25) (layer "F.Cu") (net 4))
 (segment (start 80.01 64.77) (end 80.01 82.55) (width 0.25) (layer "F.Cu") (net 4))
 (segment (start 27.94 55.88) (end 35.56 48.26) (width 0.25) (layer "F.Cu") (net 4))
 (via (at 39.37 52.07) (size 0.8) (drill 0.4) (layers "F.Cu" "B.Cu") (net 4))
 (via (at 36.83 49.53) (size 0.8) (drill 0.4) (layers "F.Cu" "B.Cu") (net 4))
 (segment (start 36.83 49.53) (end 39.37 52.07) (width 0.25) (layer "B.Cu") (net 4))
 (segment (start 27.94 50.8) (end 33.02 45.72) (width 0.25) (layer "F.Cu") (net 3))
 (segment (start 33.02 45.72) (end 33.02 29.21) (width 0.25) (layer "F.Cu") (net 3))
 (segment (start 27.94 50.8) (end 36.83 59.69) (width 0.25) (layer "B.Cu") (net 3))
 (segment (start 36.83 59.69) (end 36.83 82.55) (width 0.25) (layer "B.Cu") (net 3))
 (segment (start 50.8 68.58) (end 58.42 76.2) (width 0.25) (layer "F.Cu") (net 2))
 (segment (start 58.42 76.2) (end 58.42 82.55) (width 0.25) (layer "F.Cu") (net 2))
 (segment (start 27.94 45.72) (end 30.48 43.18) (width 0.25) (layer "F.Cu") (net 2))
 (segment (start 30.48 43.18) (end 30.48 29.21) (width 0.25) (layer "F.Cu") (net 2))
 (via (at 50.8 68.58) (size 0.8) (drill 0.4) (layers "F.Cu" "B.Cu") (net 2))
 (segment (start 27.94 45.72) (end 50.8 68.58) (width 0.25) (layer "B.Cu") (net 2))
 (segment (start 27.94 40.64) (end 27.94 29.21) (width 0.25) (layer "F.Cu") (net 1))
 (segment (start 46.99 60.96) (end 58.42 60.96) (width 0.25) (layer "F.Cu") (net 1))
 (segment (start 45.72 59.69) (end 46.99 60.96) (width 0.25) (layer "F.Cu") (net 1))
 (via (at 45.72 59.69) (size 0.8) (drill 0.4) (layers "F.Cu" "B.Cu") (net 1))
 (segment (start 27.94 40.64) (end 27.94 41.91) (width 0.25) (layer "B.Cu") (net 1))
 (segment (start 27.94 41.91) (end 45.72 59.69) (width 0.25) (layer "B.Cu") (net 1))
 (segment (start 46.355 33.02) (end 46.550153 32.824847) (width 0.25) (layer "F.Cu") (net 8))
 (segment (start 66.04 41.91) (end 49.53 41.91) (width 0.25) (layer "F.Cu") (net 8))
 (segment (start 46.355 37.555) (end 46.355 33.02) (width 0.25) (layer "F.Cu") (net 8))
 (segment (start 105.41 81.28) (end 66.04 41.91) (width 0.25) (layer "F.Cu") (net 8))
 (via (at 46.355 37.555) (size 0.8) (drill 0.4) (layers "F.Cu" "B.Cu") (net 8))
 (via (at 49.53 41.91) (size 0.8) (drill 0.4) (layers "F.Cu" "B.Cu") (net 8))
 (via (at 46.550153 32.824847) (size 0.8) (drill 0.4) (layers "F.Cu" "B.Cu") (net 8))
 (segment (start 157.48 77.47) (end 166.37 77.47) (width 0.25) (layer "B.Cu") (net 8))
 (segment (start 49.53 40.73) (end 46.355 37.555) (width 0.25) (layer "B.Cu") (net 8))
 (segment (start 45.72 31.994694) (end 45.72 29.21) (width 0.25) (layer "B.Cu") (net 8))
 (segment (start 49.53 41.91) (end 49.53 40.73) (width 0.25) (layer "B.Cu") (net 8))
 (segment (start 105.41 81.28) (end 153.67 81.28) (width 0.25) (layer "B.Cu") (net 8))
 (segment (start 153.67 81.28) (end 157.48 77.47) (width 0.25) (layer "B.Cu") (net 8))
 (segment (start 46.550153 32.824847) (end 45.72 31.994694) (width 0.25) (layer "B.Cu") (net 8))
 (segment (start 48.26 35.56) (end 52.615 39.915) (width 0.25) (layer "F.Cu") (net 7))
 (segment (start 52.615 39.915) (end 59.055 39.915) (width 0.25) (layer "F.Cu") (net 7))
 (via (at 59.055 39.915) (size 0.8) (drill 0.4) (layers "F.Cu" "B.Cu") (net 7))
 (via (at 48.26 35.56) (size 0.8) (drill 0.4) (layers "F.Cu" "B.Cu") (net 7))
 (segment (start 105.41 91.44) (end 140.97 91.44) (width 0.25) (layer "B.Cu") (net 7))
 (segment (start 43.18 30.48) (end 48.26 35.56) (width 0.25) (layer "B.Cu") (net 7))
 (segment (start 43.18 29.21) (end 43.18 30.48) (width 0.25) (layer "B.Cu") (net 7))
 (segment (start 94.615 80.645) (end 105.41 91.44) (width 0.25) (layer "B.Cu") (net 7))
 (segment (start 60.235 39.915) (end 94.615 74.295) (width 0.25) (layer "B.Cu") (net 7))
 (segment (start 59.055 39.915) (end 60.235 39.915) (width 0.25) (layer "B.Cu") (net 7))
 (segment (start 140.97 91.44) (end 144.78 95.25) (width 0.25) (layer "B.Cu") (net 7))
 (segment (start 94.615 74.295) (end 94.615 80.645) (width 0.25) (layer "B.Cu") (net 7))
 (segment (start 58.655001 39.134999) (end 54.374999 39.134999) (width 0.25) (layer "F.Cu") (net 9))
 (segment (start 54.374999 39.134999) (end 48.26 33.02) (width 0.25) (layer "F.Cu") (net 9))
 (segment (start 59.055 38.735) (end 58.655001 39.134999) (width 0.25) (layer "F.Cu") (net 9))
 (via (at 59.055 38.735) (size 0.8) (drill 0.4) (layers "F.Cu" "B.Cu") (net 9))
 (via (at 48.26 33.02) (size 0.8) (drill 0.4) (layers "F.Cu" "B.Cu") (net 9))
 (segment (start 60.325 38.735) (end 59.055 38.735) (width 0.25) (layer "B.Cu") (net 9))
 (segment (start 105.41 86.36) (end 95.885 76.835) (width 0.25) (layer "B.Cu") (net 9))
 (segment (start 95.885 76.835) (end 95.885 74.295) (width 0.25) (layer "B.Cu") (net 9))
 (segment (start 48.26 33.02) (end 48.26 29.21) (width 0.25) (layer "B.Cu") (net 9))
 (segment (start 169.545 86.36) (end 178.435 77.47) (width 0.25) (layer "B.Cu") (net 9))
 (segment (start 105.41 86.36) (end 169.545 86.36) (width 0.25) (layer "B.Cu") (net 9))
 (segment (start 178.435 77.47) (end 188.595 77.47) (width 0.25) (layer "B.Cu") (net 9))
 (segment (start 95.885 74.295) (end 60.325 38.735) (width 0.25) (layer "B.Cu") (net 9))
 (segment (start 200.025 47.625) (end 210.185 47.625) (width 0.25) (layer "F.Cu") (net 10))
 (segment (start 67.945 27.305) (end 52.705 27.305) (width 0.25) (layer "F.Cu") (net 10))
 (segment (start 69.85 29.21) (end 67.945 27.305) (width 0.25) (layer "F.Cu") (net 10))
 (segment (start 52.705 27.305) (end 50.8 29.21) (width 0.25) (layer "F.Cu") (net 10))
 (segment (start 192.584001 55.065999) (end 200.025 47.625) (width 0.25) (layer "F.Cu") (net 10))
 (segment (start 105.41 55.88) (end 106.224001 55.065999) (width 0.25) (layer "F.Cu") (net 10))
 (segment (start 106.224001 55.065999) (end 192.584001 55.065999) (width 0.25) (layer "F.Cu") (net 10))
 (via (at 69.85 29.21) (size 0.8) (drill 0.4) (layers "F.Cu" "B.Cu") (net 10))
 (segment (start 95.494999 54.854999) (end 69.85 29.21) (width 0.25) (layer "B.Cu") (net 10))
 (segment (start 105.41 55.88) (end 104.384999 54.854999) (width 0.25) (layer "B.Cu") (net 10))
 (segment (start 104.384999 54.854999) (end 95.494999 54.854999) (width 0.25) (layer "B.Cu") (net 10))
 (segment (start 64.045 39.915) (end 65.405 39.915) (width 0.25) (layer "F.Cu") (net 11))
 (segment (start 58.42 34.29) (end 64.045 39.915) (width 0.25) (layer "F.Cu") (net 11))
 (via (at 58.42 34.29) (size 0.8) (drill 0.4) (layers "F.Cu" "B.Cu") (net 11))
 (via (at 65.405 39.915) (size 0.8) (drill 0.4) (layers "F.Cu" "B.Cu") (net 11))
 (segment (start 105.41 71.12) (end 118.745 71.12) (width 0.25) (layer "B.Cu") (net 11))
 (segment (start 65.405 39.915) (end 74.205 39.915) (width 0.25) (layer "B.Cu") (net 11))
 (segment (start 118.745 71.12) (end 133.35 56.515) (width 0.25) (layer "B.Cu") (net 11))
 (segment (start 74.205 39.915) (end 105.41 71.12) (width 0.25) (layer "B.Cu") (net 11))
 (segment (start 53.34 29.21) (end 58.42 34.29) (width 0.25) (layer "B.Cu") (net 11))
 (segment (start 133.35 56.515) (end 144.78 56.515) (width 0.25) (layer "B.Cu") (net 11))
 (segment (start 60.325 33.655) (end 66.04 39.37) (width 0.25) (layer "F.Cu") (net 12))
 (segment (start 66.04 39.37) (end 74.93 39.37) (width 0.25) (layer "F.Cu") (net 12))
 (via (at 74.93 39.37) (size 0.8) (drill 0.4) (layers "F.Cu" "B.Cu") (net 12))
 (via (at 60.325 33.655) (size 0.8) (drill 0.4) (layers "F.Cu" "B.Cu") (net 12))
 (segment (start 74.93 39.37) (end 94.615 59.055) (width 0.25) (layer "B.Cu") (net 12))
 (segment (start 103.505 59.055) (end 105.41 60.96) (width 0.25) (layer "B.Cu") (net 12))
 (segment (start 137.16 38.735) (end 166.37 38.735) (width 0.25) (layer "B.Cu") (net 12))
 (segment (start 94.615 59.055) (end 103.505 59.055) (width 0.25) (layer "B.Cu") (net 12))
 (segment (start 114.935 60.96) (end 137.16 38.735) (width 0.25) (layer "B.Cu") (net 12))
 (segment (start 55.88 29.21) (end 60.325 33.655) (width 0.25) (layer "B.Cu") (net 12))
 (segment (start 105.41 60.96) (end 114.935 60.96) (width 0.25) (layer "B.Cu") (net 12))
 (segment (start 61.399847 32.824847) (end 67.31 38.735) (width 0.25) (layer "F.Cu") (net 13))
 (segment (start 94.525 55.155) (end 105.41 66.04) (width 0.25) (layer "F.Cu") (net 13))
 (segment (start 76.744999 38.644999) (end 76.835 38.735) (width 0.25) (layer "F.Cu") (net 13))
 (segment (start 67.31 38.735) (end 67.400001 38.644999) (width 0.25) (layer "F.Cu") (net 13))
 (segment (start 93.345 55.155) (end 94.525 55.155) (width 0.25) (layer "F.Cu") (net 13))
 (segment (start 67.400001 38.644999) (end 76.744999 38.644999) (width 0.25) (layer "F.Cu") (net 13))
 (via (at 93.345 55.155) (size 0.8) (drill 0.4) (layers "F.Cu" "B.Cu") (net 13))
 (via (at 61.399847 32.824847) (size 0.8) (drill 0.4) (layers "F.Cu" "B.Cu") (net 13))
 (via (at 76.835 38.735) (size 0.8) (drill 0.4) (layers "F.Cu" "B.Cu") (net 13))
 (segment (start 76.835 38.735) (end 93.255 55.155) (width 0.25) (layer "B.Cu") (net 13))
 (segment (start 135.255 48.26) (end 167.005 48.26) (width 0.25) (layer "B.Cu") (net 13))
 (segment (start 117.475 66.04) (end 135.255 48.26) (width 0.25) (layer "B.Cu") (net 13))
 (segment (start 105.41 66.04) (end 117.475 66.04) (width 0.25) (layer "B.Cu") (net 13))
 (segment (start 93.255 55.155) (end 93.345 55.155) (width 0.25) (layer "B.Cu") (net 13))
 (segment (start 167.005 48.26) (end 176.53 38.735) (width 0.25) (layer "B.Cu") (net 13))
 (segment (start 58.42 29.21) (end 61.399847 32.189847) (width 0.25) (layer "B.Cu") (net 13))
 (segment (start 176.53 38.735) (end 188.595 38.735) (width 0.25) (layer "B.Cu") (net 13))
 (segment (start 61.399847 32.189847) (end 61.399847 32.824847) (width 0.25) (layer "B.Cu") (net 13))
 (segment (start 53.34 31.025) (end 59.145 31.025) (width 0.25) (layer "F.Cu") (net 14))
 (segment (start 59.145 31.025) (end 60.96 29.21) (width 0.25) (layer "F.Cu") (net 14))
 (segment (start 61.595 38.735) (end 60.87 38.735) (width 0.25) (layer "F.Cu") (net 14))
 (segment (start 60.87 38.735) (end 54.61 32.475) (width 0.25) (layer "F.Cu") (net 14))
 (via (at 54.61 32.475) (size 0.8) (drill 0.4) (layers "F.Cu" "B.Cu") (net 14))
 (via (at 61.595 38.735) (size 0.8) (drill 0.4) (layers "F.Cu" "B.Cu") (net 14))
 (via (at 53.34 31.025) (size 0.8) (drill 0.4) (layers "F.Cu" "B.Cu") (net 14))
 (segment (start 54.61 32.475) (end 54.61 32.295) (width 0.25) (layer "B.Cu") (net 14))
 (segment (start 105.41 76.2) (end 70.485 41.275) (width 0.25) (layer "B.Cu") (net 14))
 (segment (start 125.73 76.2) (end 129.54 72.39) (width 0.25) (layer "B.Cu") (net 14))
 (segment (start 70.485 41.275) (end 64.135 41.275) (width 0.25) (layer "B.Cu") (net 14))
 (segment (start 64.135 41.275) (end 61.595 38.735) (width 0.25) (layer "B.Cu") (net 14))
 (segment (start 54.61 32.295) (end 53.34 31.025) (width 0.25) (layer "B.Cu") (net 14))
 (segment (start 105.41 76.2) (end 125.73 76.2) (width 0.25) (layer "B.Cu") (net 14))
 (segment (start 129.54 72.39) (end 196.215 72.39) (width 0.25) (layer "B.Cu") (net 14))
 (segment (start 196.215 72.39) (end 210.185 86.36) (width 0.25) (layer "B.Cu") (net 14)))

